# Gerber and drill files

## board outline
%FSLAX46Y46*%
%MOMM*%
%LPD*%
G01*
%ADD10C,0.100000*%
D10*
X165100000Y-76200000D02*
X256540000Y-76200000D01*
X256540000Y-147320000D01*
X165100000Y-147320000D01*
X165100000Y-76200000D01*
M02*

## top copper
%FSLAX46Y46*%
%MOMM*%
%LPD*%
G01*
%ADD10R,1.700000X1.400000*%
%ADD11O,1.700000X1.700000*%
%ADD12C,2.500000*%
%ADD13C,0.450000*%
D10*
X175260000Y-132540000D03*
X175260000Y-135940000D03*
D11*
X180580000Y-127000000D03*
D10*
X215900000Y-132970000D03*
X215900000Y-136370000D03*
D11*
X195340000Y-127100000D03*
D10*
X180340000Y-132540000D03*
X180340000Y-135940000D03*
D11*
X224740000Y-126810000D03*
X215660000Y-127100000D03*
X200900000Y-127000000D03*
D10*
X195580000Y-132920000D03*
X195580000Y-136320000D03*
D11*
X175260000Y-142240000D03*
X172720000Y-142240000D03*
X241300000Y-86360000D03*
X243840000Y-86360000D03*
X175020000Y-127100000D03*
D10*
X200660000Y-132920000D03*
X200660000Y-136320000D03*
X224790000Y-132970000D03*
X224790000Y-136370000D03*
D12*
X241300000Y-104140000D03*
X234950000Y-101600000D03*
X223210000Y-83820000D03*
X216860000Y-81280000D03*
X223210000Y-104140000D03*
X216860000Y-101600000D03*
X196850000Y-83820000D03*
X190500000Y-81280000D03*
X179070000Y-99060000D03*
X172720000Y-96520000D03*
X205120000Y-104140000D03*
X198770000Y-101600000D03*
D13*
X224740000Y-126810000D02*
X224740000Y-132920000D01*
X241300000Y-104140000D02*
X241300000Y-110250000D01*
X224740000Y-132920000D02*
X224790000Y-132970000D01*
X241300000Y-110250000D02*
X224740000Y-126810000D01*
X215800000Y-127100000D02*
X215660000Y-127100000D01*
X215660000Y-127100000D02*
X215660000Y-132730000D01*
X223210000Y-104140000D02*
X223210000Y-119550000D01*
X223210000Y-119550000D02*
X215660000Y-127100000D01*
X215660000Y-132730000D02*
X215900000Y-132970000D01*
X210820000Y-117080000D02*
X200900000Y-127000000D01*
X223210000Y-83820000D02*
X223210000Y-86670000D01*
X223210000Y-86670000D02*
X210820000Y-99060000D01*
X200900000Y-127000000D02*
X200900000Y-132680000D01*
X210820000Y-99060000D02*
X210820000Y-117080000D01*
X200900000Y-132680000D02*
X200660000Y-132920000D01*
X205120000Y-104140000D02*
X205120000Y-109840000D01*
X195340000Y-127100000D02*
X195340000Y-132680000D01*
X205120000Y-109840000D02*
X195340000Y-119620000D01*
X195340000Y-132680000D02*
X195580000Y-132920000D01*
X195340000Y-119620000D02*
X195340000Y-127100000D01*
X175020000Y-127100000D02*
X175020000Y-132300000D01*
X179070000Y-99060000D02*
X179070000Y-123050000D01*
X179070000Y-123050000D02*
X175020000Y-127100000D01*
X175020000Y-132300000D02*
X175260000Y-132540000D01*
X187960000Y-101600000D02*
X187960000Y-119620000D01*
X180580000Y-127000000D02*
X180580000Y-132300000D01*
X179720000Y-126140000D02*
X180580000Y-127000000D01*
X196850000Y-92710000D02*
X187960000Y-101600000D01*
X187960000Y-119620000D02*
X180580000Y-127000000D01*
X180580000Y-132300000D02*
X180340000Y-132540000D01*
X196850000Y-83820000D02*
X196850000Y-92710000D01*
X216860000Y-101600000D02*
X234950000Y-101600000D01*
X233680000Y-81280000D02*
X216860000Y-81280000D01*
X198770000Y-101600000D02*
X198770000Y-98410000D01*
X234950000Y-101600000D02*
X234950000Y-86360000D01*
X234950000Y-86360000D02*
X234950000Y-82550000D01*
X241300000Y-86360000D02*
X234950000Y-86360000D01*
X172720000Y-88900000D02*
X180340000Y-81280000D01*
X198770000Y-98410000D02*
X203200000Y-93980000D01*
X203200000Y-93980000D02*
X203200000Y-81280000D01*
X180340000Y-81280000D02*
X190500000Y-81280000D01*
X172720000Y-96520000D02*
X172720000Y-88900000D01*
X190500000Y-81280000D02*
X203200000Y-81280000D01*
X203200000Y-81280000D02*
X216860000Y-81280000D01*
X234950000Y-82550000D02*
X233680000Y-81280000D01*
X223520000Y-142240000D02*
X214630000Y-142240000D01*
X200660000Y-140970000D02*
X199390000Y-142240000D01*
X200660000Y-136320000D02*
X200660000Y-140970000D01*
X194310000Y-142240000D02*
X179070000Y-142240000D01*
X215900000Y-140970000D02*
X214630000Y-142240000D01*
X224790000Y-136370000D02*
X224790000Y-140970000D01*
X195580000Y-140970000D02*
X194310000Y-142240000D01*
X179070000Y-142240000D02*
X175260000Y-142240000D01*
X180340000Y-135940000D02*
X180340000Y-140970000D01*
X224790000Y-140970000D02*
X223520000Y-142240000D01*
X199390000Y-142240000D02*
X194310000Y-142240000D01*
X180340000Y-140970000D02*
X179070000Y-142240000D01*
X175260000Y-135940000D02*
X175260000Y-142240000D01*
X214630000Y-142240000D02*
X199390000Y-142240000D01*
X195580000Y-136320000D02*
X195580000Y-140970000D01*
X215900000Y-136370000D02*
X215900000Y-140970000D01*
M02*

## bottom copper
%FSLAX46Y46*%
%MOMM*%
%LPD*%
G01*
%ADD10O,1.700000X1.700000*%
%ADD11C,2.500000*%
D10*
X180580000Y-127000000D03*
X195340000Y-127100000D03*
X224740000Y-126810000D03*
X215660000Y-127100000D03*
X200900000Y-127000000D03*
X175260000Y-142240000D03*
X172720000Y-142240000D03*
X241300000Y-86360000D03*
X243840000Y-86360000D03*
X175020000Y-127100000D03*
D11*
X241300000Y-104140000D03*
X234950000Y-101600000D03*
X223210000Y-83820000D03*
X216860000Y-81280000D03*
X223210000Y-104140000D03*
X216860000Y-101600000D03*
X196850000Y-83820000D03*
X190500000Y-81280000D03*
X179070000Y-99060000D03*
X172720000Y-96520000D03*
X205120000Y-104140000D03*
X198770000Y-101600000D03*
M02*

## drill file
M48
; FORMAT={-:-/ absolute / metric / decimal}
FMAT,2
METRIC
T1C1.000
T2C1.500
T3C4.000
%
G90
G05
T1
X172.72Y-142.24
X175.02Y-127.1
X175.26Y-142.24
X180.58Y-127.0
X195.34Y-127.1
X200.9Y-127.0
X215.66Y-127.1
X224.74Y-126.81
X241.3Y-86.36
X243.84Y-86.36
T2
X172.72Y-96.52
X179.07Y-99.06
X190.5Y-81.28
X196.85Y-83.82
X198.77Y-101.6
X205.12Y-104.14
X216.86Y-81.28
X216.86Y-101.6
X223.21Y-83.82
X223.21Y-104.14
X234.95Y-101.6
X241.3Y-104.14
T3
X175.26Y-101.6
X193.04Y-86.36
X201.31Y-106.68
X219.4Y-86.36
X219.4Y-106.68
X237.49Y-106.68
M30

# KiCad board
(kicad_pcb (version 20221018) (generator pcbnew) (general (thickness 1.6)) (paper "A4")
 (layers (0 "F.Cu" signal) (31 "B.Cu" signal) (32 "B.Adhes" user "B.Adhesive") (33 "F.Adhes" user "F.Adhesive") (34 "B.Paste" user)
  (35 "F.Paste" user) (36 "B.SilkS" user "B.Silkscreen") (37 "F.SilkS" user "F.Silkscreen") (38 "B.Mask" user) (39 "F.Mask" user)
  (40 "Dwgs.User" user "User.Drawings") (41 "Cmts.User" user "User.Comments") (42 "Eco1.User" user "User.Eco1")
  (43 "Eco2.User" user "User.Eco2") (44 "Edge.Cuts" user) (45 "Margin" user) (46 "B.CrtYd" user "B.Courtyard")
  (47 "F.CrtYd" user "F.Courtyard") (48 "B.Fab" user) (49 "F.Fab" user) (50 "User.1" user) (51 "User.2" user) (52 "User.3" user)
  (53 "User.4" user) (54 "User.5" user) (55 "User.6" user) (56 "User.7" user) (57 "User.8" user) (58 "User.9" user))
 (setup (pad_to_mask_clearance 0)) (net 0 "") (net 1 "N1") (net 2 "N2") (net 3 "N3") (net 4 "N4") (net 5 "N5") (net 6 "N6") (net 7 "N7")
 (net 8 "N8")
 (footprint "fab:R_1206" (layer "F.Cu") (at 175.26 134.24 -90)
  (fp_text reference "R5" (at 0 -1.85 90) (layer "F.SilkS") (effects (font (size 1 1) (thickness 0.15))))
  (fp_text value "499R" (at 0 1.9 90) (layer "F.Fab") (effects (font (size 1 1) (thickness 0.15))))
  (pad "1" smd rect (at -1.7 0 270) (size 1.4 1.7) (layers "F.Cu" "F.Paste" "F.Mask") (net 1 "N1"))
  (pad "2" smd rect (at 1.7 0 270) (size 1.4 1.7) (layers "F.Cu" "F.Paste" "F.Mask") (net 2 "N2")))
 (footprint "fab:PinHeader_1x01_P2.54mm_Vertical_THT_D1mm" (layer "F.Cu") (at 180.58 127)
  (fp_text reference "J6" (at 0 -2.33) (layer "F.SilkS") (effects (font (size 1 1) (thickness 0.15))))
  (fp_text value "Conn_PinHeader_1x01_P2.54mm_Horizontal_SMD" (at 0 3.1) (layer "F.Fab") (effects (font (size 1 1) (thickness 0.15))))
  (pad "1" thru_hole oval (at 0 0) (size 1.7 1.7) (drill 1) (layers "*.Cu" "*.Mask") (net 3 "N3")))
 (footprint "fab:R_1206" (layer "F.Cu") (at 215.9 134.67 -90)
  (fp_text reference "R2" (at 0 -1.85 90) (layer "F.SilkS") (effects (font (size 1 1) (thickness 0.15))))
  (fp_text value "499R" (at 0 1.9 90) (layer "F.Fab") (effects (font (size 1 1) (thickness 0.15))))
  (pad "1" smd rect (at -1.7 0 270) (size 1.4 1.7) (layers "F.Cu" "F.Paste" "F.Mask") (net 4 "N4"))
  (pad "2" smd rect (at 1.7 0 270) (size 1.4 1.7) (layers "F.Cu" "F.Paste" "F.Mask") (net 2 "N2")))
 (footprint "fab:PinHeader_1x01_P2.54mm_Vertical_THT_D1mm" (layer "F.Cu") (at 195.34 127.1 180)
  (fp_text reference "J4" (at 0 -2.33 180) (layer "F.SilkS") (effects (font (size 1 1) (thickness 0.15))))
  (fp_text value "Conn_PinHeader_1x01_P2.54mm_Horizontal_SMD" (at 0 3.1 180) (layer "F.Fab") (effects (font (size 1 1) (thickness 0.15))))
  (pad "1" thru_hole oval (at 0 0 180) (size 1.7 1.7) (drill 1) (layers "*.Cu" "*.Mask") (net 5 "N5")))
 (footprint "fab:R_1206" (layer "F.Cu") (at 180.34 134.24 -90)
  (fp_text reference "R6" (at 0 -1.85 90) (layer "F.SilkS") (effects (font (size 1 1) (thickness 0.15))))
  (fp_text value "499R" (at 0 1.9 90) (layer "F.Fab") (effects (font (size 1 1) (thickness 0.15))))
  (pad "1" smd rect (at -1.7 0 270) (size 1.4 1.7) (layers "F.Cu" "F.Paste" "F.Mask") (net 3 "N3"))
  (pad "2" smd rect (at 1.7 0 270) (size 1.4 1.7) (layers "F.Cu" "F.Paste" "F.Mask") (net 2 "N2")))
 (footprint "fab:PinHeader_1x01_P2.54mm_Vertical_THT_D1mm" (layer "F.Cu") (at 224.74 126.81)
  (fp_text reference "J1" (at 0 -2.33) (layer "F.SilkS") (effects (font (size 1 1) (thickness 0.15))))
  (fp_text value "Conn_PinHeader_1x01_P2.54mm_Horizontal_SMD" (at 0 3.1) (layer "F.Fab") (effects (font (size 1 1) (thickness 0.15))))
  (pad "1" thru_hole oval (at 0 0) (size 1.7 1.7) (drill 1) (layers "*.Cu" "*.Mask") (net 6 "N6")))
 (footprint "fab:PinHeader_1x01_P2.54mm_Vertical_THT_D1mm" (layer "F.Cu") (at 215.66 127.1 180)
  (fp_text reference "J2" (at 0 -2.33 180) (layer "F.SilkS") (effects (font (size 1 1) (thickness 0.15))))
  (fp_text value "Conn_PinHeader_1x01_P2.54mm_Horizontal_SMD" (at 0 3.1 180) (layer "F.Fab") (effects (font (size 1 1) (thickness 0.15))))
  (pad "1" thru_hole oval (at 0 0 180) (size 1.7 1.7) (drill 1) (layers "*.Cu" "*.Mask") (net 4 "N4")))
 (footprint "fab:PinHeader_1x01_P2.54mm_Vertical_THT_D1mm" (layer "F.Cu") (at 200.9 127)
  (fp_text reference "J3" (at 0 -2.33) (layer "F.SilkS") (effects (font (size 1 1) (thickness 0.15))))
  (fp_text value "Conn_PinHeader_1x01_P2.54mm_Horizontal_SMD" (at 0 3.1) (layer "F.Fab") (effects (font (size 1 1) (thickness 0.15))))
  (pad "1" thru_hole oval (at 0 0) (size 1.7 1.7) (drill 1) (layers "*.Cu" "*.Mask") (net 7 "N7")))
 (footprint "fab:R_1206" (layer "F.Cu") (at 195.58 134.62 -90)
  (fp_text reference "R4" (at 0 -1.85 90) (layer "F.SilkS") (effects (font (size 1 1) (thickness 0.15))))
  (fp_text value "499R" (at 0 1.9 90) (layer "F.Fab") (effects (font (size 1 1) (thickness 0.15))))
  (pad "1" smd rect (at -1.7 0 270) (size 1.4 1.7) (layers "F.Cu" "F.Paste" "F.Mask") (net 5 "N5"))
  (pad "2" smd rect (at 1.7 0 270) (size 1.4 1.7) (layers "F.Cu" "F.Paste" "F.Mask") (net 2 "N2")))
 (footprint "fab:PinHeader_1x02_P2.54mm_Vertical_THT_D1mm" (layer "F.Cu") (at 175.26 142.24 -90)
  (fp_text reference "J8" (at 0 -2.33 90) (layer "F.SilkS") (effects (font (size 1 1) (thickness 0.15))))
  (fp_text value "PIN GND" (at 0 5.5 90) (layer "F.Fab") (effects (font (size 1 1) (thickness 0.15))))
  (pad "1" thru_hole oval (at 0 0 270) (size 1.7 1.7) (drill 1) (layers "*.Cu" "*.Mask") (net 2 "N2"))
  (pad "2" thru_hole oval (at 0 2.54 270) (size 1.7 1.7) (drill 1) (layers "*.Cu" "*.Mask")))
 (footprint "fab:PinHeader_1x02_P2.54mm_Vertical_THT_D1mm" (layer "F.Cu") (at 241.3 86.36 90)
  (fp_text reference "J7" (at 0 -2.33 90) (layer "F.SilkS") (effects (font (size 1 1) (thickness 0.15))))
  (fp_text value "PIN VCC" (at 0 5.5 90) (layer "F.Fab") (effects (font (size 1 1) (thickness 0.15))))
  (pad "1" thru_hole oval (at 0 0 90) (size 1.7 1.7) (drill 1) (layers "*.Cu" "*.Mask") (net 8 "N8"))
  (pad "2" thru_hole oval (at 0 2.54 90) (size 1.7 1.7) (drill 1) (layers "*.Cu" "*.Mask")))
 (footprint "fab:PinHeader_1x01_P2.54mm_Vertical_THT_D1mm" (layer "F.Cu") (at 175.02 127.1 180)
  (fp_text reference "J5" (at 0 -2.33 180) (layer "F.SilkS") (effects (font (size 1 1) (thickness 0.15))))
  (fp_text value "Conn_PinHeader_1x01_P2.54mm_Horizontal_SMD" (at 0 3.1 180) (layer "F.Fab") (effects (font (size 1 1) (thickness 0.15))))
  (pad "1" thru_hole oval (at 0 0 180) (size 1.7 1.7) (drill 1) (layers "*.Cu" "*.Mask") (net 1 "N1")))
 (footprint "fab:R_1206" (layer "F.Cu") (at 200.66 134.62 -90)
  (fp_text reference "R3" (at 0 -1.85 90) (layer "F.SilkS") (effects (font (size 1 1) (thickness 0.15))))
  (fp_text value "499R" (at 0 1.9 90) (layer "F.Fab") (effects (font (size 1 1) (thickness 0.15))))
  (pad "1" smd rect (at -1.7 0 270) (size 1.4 1.7) (layers "F.Cu" "F.Paste" "F.Mask") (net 7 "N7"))
  (pad "2" smd rect (at 1.7 0 270) (size 1.4 1.7) (layers "F.Cu" "F.Paste" "F.Mask") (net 2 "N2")))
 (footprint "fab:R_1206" (layer "F.Cu") (at 224.79 134.67 -90)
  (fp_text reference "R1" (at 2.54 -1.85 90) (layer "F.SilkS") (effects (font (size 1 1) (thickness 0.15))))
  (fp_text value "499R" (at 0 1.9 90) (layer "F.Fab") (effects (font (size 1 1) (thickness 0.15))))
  (pad "1" smd rect (at -1.7 0 270) (size 1.4 1.7) (layers "F.Cu" "F.Paste" "F.Mask") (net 6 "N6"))
  (pad "2" smd rect (at 1.7 0 270) (size 1.4 1.7) (layers "F.Cu" "F.Paste" "F.Mask") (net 2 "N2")))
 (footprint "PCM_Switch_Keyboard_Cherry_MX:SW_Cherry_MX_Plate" (layer "B.Cu") (at 237.49 106.68 180)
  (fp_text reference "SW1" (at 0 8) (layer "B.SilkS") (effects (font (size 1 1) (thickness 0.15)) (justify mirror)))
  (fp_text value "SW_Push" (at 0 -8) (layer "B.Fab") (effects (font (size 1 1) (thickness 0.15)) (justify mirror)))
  (pad "" np_thru_hole circle (at 0 0 180) (size 4 4) (drill 4) (layers "*.Cu" "*.Mask"))
  (pad "1" thru_hole circle (at -3.81 2.54 180) (size 2.5 2.5) (drill 1.5) (layers "*.Cu" "*.Mask") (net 6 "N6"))
  (pad "2" thru_hole circle (at 2.54 5.08 180) (size 2.5 2.5) (drill 1.5) (layers "*.Cu" "*.Mask") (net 8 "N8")))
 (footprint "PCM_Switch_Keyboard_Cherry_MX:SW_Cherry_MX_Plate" (layer "B.Cu") (at 219.4 86.36 180)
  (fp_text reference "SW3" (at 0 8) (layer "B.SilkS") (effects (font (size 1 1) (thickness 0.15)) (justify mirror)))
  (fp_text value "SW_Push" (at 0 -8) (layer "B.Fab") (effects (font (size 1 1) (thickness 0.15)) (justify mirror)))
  (pad "" np_thru_hole circle (at 0 0 180) (size 4 4) (drill 4) (layers "*.Cu" "*.Mask"))
  (pad "1" thru_hole circle (at -3.81 2.54 180) (size 2.5 2.5) (drill 1.5) (layers "*.Cu" "*.Mask") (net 7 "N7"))
  (pad "2" thru_hole circle (at 2.54 5.08 180) (size 2.5 2.5) (drill 1.5) (layers "*.Cu" "*.Mask") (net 8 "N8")))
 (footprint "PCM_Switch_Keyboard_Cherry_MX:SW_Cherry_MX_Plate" (layer "B.Cu") (at 219.4 106.68 180)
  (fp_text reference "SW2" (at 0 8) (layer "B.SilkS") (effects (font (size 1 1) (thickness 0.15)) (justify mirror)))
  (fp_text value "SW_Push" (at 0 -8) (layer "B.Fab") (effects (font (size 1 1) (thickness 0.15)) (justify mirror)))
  (pad "" np_thru_hole circle (at 0 0 180) (size 4 4) (drill 4) (layers "*.Cu" "*.Mask"))
  (pad "1" thru_hole circle (at -3.81 2.54 180) (size 2.5 2.5) (drill 1.5) (layers "*.Cu" "*.Mask") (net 4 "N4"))
  (pad "2" thru_hole circle (at 2.54 5.08 180) (size 2.5 2.5) (drill 1.5) (layers "*.Cu" "*.Mask") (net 8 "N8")))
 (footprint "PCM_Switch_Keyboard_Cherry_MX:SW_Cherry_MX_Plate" (layer "B.Cu") (at 193.04 86.36 180)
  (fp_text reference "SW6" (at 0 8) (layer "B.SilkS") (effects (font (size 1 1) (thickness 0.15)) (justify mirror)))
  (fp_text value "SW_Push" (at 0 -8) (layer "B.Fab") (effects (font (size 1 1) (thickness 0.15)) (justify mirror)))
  (pad "" np_thru_hole circle (at 0 0 180) (size 4 4) (drill 4) (layers "*.Cu" "*.Mask"))
  (pad "1" thru_hole circle (at -3.81 2.54 180) (size 2.5 2.5) (drill 1.5) (layers "*.Cu" "*.Mask") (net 3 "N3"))
  (pad "2" thru_hole circle (at 2.54 5.08 180) (size 2.5 2.5) (drill 1.5) (layers "*.Cu" "*.Mask") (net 8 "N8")))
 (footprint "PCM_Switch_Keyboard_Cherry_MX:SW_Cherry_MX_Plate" (layer "B.Cu") (at 175.26 101.6 180)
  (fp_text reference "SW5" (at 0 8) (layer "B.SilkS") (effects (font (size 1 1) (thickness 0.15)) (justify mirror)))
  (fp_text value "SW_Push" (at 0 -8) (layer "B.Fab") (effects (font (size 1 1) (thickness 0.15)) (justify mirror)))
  (pad "" np_thru_hole circle (at 0 0 180) (size 4 4) (drill 4) (layers "*.Cu" "*.Mask"))
  (pad "1" thru_hole circle (at -3.81 2.54 180) (size 2.5 2.5) (drill 1.5) (layers "*.Cu" "*.Mask") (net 1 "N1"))
  (pad "2" thru_hole circle (at 2.54 5.08 180) (size 2.5 2.5) (drill 1.5) (layers "*.Cu" "*.Mask") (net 8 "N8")))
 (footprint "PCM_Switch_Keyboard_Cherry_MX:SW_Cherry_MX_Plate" (layer "B.Cu") (at 201.31 106.68 180)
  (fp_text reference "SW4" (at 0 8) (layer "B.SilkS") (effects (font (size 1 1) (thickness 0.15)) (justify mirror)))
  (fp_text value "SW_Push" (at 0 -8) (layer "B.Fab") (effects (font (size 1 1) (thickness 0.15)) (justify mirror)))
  (pad "" np_thru_hole circle (at 0 0 180) (size 4 4) (drill 4) (layers "*.Cu" "*.Mask"))
  (pad "1" thru_hole circle (at -3.81 2.54 180) (size 2.5 2.5) (drill 1.5) (layers "*.Cu" "*.Mask") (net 5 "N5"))
  (pad "2" thru_hole circle (at 2.54 5.08 180) (size 2.5 2.5) (drill 1.5) (layers "*.Cu" "*.Mask") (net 8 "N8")))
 (gr_rect (start 165.1 76.2) (end 256.54 147.32) (stroke (width 0.1) (type default)) (fill none) (layer "Edge.Cuts"))
 (segment (start 224.74 126.81) (end 224.74 132.92) (width 0.45) (layer "F.Cu") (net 6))
 (segment (start 241.3 104.14) (end 241.3 110.25) (width 0.45) (layer "F.Cu") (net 6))
 (segment (start 224.74 132.92) (end 224.79 132.97) (width 0.45) (layer "F.Cu") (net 6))
 (segment (start 241.3 110.25) (end 224.74 126.81) (width 0.45) (layer "F.Cu") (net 6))
 (segment (start 215.8 127.1) (end 215.66 127.1) (width 0.45) (layer "F.Cu") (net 4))
 (segment (start 215.66 127.1) (end 215.66 132.73) (width 0.45) (layer "F.Cu") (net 4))
 (segment (start 223.21 104.14) (end 223.21 119.55) (width 0.45) (layer "F.Cu") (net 4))
 (segment (start 223.21 119.55) (end 215.66 127.1) (width 0.45) (layer "F.Cu") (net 4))
 (segment (start 215.66 132.73) (end 215.9 132.97) (width 0.45) (layer "F.Cu") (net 4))
 (segment (start 210.82 117.08) (end 200.9 127) (width 0.45) (layer "F.Cu") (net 7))
 (segment (start 223.21 83.82) (end 223.21 86.67) (width 0.45) (layer "F.Cu") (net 7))
 (segment (start 223.21 86.67) (end 210.82 99.06) (width 0.45) (layer "F.Cu") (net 7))
 (segment (start 200.9 127) (end 200.9 132.68) (width 0.45) (layer "F.Cu") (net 7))
 (segment (start 210.82 99.06) (end 210.82 117.08) (width 0.45) (layer "F.Cu") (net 7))
 (segment (start 200.9 132.68) (end 200.66 132.92) (width 0.45) (layer "F.Cu") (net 7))
 (segment (start 205.12 104.14) (end 205.12 109.84) (width 0.45) (layer "F.Cu") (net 5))
 (segment (start 195.34 127.1) (end 195.34 132.68) (width 0.45) (layer "F.Cu") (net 5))
 (segment (start 205.12 109.84) (end 195.34 119.62) (width 0.45) (layer "F.Cu") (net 5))
 (segment (start 195.34 132.68) (end 195.58 132.92) (width 0.45) (layer "F.Cu") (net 5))
 (segment (start 195.34 119.62) (end 195.34 127.1) (width 0.45) (layer "F.Cu") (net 5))
 (segment (start 175.02 127.1) (end 175.02 132.3) (width 0.45) (layer "F.Cu") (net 1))
 (segment (start 179.07 99.06) (end 179.07 123.05) (width 0.45) (layer "F.Cu") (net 1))
 (segment (start 179.07 123.05) (end 175.02 127.1) (width 0.45) (layer "F.Cu") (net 1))
 (segment (start 175.02 132.3) (end 175.26 132.54) (width 0.45) (layer "F.Cu") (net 1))
 (segment (start 187.96 101.6) (end 187.96 119.62) (width 0.45) (layer "F.Cu") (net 3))
 (segment (start 180.58 127) (end 180.58 132.3) (width 0.45) (layer "F.Cu") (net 3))
 (segment (start 179.72 126.14) (end 180.58 127) (width 0.45) (layer "F.Cu") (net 3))
 (segment (start 196.85 92.71) (end 187.96 101.6) (width 0.45) (layer "F.Cu") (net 3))
 (segment (start 187.96 119.62) (end 180.58 127) (width 0.45) (layer "F.Cu") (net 3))
 (segment (start 180.58 132.3) (end 180.34 132.54) (width 0.45) (layer "F.Cu") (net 3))
 (segment (start 196.85 83.82) (end 196.85 92.71) (width 0.45) (layer "F.Cu") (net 3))
 (segment (start 216.86 101.6) (end 234.95 101.6) (width 0.45) (layer "F.Cu") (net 8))
 (segment (start 233.68 81.28) (end 216.86 81.28) (width 0.45) (layer "F.Cu") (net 8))
 (segment (start 198.77 101.6) (end 198.77 98.41) (width 0.45) (layer "F.Cu") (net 8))
 (segment (start 234.95 101.6) (end 234.95 86.36) (width 0.45) (layer "F.Cu") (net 8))
 (segment (start 234.95 86.36) (end 234.95 82.55) (width 0.45) (layer "F.Cu") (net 8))
 (segment (start 241.3 86.36) (end 234.95 86.36) (width 0.45) (layer "F.Cu") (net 8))
 (segment (start 172.72 88.9) (end 180.34 81.28) (width 0.45) (layer "F.Cu") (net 8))
 (segment (start 198.77 98.41) (end 203.2 93.98) (width 0.45) (layer "F.Cu") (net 8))
 (segment (start 203.2 93.98) (end 203.2 81.28) (width 0.45) (layer "F.Cu") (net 8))
 (segment (start 180.34 81.28) (end 190.5 81.28) (width 0.45) (layer "F.Cu") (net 8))
 (segment (start 172.72 96.52) (end 172.72 88.9) (width 0.45) (layer "F.Cu") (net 8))
 (segment (start 190.5 81.28) (end 203.2 81.28) (width 0.45) (layer "F.Cu") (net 8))
 (segment (start 203.2 81.28) (end 216.86 81.28) (width 0.45) (layer "F.Cu") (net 8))
 (segment (start 234.95 82.55) (end 233.68 81.28) (width 0.45) (layer "F.Cu") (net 8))
 (segment (start 223.52 142.24) (end 214.63 142.24) (width 0.45) (layer "F.Cu") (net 2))
 (segment (start 200.66 140.97) (end 199.39 142.24) (width 0.45) (layer "F.Cu") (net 2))
 (segment (start 200.66 136.32) (end 200.66 140.97) (width 0.45) (layer "F.Cu") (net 2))
 (segment (start 194.31 142.24) (end 179.07 142.24) (width 0.45) (layer "F.Cu") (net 2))
 (segment (start 215.9 140.97) (end 214.63 142.24) (width 0.45) (layer "F.Cu") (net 2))
 (segment (start 224.79 136.37) (end 224.79 140.97) (width 0.45) (layer "F.Cu") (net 2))
 (segment (start 195.58 140.97) (end 194.31 142.24) (width 0.45) (layer "F.Cu") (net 2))
 (segment (start 179.07 142.24) (end 175.26 142.24) (width 0.45) (layer "F.Cu") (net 2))
 (segment (start 180.34 135.94) (end 180.34 140.97) (width 0.45) (layer "F.Cu") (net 2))
 (segment (start 224.79 140.97) (end 223.52 142.24) (width 0.45) (layer "F.Cu") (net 2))
 (segment (start 199.39 142.24) (end 194.31 142.24) (width 0.45) (layer "F.Cu") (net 2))
 (segment (start 180.34 140.97) (end 179.07 142.24) (width 0.45) (layer "F.Cu") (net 2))
 (segment (start 175.26 135.94) (end 175.26 142.24) (width 0.45) (layer "F.Cu") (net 2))
 (segment (start 214.63 142.24) (end 199.39 142.24) (width 0.45) (layer "F.Cu") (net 2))
 (segment (start 195.58 136.32) (end 195.58 140.97) (width 0.45) (layer "F.Cu") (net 2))
 (segment (start 215.9 136.37) (end 215.9 140.97) (width 0.45) (layer "F.Cu") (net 2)))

